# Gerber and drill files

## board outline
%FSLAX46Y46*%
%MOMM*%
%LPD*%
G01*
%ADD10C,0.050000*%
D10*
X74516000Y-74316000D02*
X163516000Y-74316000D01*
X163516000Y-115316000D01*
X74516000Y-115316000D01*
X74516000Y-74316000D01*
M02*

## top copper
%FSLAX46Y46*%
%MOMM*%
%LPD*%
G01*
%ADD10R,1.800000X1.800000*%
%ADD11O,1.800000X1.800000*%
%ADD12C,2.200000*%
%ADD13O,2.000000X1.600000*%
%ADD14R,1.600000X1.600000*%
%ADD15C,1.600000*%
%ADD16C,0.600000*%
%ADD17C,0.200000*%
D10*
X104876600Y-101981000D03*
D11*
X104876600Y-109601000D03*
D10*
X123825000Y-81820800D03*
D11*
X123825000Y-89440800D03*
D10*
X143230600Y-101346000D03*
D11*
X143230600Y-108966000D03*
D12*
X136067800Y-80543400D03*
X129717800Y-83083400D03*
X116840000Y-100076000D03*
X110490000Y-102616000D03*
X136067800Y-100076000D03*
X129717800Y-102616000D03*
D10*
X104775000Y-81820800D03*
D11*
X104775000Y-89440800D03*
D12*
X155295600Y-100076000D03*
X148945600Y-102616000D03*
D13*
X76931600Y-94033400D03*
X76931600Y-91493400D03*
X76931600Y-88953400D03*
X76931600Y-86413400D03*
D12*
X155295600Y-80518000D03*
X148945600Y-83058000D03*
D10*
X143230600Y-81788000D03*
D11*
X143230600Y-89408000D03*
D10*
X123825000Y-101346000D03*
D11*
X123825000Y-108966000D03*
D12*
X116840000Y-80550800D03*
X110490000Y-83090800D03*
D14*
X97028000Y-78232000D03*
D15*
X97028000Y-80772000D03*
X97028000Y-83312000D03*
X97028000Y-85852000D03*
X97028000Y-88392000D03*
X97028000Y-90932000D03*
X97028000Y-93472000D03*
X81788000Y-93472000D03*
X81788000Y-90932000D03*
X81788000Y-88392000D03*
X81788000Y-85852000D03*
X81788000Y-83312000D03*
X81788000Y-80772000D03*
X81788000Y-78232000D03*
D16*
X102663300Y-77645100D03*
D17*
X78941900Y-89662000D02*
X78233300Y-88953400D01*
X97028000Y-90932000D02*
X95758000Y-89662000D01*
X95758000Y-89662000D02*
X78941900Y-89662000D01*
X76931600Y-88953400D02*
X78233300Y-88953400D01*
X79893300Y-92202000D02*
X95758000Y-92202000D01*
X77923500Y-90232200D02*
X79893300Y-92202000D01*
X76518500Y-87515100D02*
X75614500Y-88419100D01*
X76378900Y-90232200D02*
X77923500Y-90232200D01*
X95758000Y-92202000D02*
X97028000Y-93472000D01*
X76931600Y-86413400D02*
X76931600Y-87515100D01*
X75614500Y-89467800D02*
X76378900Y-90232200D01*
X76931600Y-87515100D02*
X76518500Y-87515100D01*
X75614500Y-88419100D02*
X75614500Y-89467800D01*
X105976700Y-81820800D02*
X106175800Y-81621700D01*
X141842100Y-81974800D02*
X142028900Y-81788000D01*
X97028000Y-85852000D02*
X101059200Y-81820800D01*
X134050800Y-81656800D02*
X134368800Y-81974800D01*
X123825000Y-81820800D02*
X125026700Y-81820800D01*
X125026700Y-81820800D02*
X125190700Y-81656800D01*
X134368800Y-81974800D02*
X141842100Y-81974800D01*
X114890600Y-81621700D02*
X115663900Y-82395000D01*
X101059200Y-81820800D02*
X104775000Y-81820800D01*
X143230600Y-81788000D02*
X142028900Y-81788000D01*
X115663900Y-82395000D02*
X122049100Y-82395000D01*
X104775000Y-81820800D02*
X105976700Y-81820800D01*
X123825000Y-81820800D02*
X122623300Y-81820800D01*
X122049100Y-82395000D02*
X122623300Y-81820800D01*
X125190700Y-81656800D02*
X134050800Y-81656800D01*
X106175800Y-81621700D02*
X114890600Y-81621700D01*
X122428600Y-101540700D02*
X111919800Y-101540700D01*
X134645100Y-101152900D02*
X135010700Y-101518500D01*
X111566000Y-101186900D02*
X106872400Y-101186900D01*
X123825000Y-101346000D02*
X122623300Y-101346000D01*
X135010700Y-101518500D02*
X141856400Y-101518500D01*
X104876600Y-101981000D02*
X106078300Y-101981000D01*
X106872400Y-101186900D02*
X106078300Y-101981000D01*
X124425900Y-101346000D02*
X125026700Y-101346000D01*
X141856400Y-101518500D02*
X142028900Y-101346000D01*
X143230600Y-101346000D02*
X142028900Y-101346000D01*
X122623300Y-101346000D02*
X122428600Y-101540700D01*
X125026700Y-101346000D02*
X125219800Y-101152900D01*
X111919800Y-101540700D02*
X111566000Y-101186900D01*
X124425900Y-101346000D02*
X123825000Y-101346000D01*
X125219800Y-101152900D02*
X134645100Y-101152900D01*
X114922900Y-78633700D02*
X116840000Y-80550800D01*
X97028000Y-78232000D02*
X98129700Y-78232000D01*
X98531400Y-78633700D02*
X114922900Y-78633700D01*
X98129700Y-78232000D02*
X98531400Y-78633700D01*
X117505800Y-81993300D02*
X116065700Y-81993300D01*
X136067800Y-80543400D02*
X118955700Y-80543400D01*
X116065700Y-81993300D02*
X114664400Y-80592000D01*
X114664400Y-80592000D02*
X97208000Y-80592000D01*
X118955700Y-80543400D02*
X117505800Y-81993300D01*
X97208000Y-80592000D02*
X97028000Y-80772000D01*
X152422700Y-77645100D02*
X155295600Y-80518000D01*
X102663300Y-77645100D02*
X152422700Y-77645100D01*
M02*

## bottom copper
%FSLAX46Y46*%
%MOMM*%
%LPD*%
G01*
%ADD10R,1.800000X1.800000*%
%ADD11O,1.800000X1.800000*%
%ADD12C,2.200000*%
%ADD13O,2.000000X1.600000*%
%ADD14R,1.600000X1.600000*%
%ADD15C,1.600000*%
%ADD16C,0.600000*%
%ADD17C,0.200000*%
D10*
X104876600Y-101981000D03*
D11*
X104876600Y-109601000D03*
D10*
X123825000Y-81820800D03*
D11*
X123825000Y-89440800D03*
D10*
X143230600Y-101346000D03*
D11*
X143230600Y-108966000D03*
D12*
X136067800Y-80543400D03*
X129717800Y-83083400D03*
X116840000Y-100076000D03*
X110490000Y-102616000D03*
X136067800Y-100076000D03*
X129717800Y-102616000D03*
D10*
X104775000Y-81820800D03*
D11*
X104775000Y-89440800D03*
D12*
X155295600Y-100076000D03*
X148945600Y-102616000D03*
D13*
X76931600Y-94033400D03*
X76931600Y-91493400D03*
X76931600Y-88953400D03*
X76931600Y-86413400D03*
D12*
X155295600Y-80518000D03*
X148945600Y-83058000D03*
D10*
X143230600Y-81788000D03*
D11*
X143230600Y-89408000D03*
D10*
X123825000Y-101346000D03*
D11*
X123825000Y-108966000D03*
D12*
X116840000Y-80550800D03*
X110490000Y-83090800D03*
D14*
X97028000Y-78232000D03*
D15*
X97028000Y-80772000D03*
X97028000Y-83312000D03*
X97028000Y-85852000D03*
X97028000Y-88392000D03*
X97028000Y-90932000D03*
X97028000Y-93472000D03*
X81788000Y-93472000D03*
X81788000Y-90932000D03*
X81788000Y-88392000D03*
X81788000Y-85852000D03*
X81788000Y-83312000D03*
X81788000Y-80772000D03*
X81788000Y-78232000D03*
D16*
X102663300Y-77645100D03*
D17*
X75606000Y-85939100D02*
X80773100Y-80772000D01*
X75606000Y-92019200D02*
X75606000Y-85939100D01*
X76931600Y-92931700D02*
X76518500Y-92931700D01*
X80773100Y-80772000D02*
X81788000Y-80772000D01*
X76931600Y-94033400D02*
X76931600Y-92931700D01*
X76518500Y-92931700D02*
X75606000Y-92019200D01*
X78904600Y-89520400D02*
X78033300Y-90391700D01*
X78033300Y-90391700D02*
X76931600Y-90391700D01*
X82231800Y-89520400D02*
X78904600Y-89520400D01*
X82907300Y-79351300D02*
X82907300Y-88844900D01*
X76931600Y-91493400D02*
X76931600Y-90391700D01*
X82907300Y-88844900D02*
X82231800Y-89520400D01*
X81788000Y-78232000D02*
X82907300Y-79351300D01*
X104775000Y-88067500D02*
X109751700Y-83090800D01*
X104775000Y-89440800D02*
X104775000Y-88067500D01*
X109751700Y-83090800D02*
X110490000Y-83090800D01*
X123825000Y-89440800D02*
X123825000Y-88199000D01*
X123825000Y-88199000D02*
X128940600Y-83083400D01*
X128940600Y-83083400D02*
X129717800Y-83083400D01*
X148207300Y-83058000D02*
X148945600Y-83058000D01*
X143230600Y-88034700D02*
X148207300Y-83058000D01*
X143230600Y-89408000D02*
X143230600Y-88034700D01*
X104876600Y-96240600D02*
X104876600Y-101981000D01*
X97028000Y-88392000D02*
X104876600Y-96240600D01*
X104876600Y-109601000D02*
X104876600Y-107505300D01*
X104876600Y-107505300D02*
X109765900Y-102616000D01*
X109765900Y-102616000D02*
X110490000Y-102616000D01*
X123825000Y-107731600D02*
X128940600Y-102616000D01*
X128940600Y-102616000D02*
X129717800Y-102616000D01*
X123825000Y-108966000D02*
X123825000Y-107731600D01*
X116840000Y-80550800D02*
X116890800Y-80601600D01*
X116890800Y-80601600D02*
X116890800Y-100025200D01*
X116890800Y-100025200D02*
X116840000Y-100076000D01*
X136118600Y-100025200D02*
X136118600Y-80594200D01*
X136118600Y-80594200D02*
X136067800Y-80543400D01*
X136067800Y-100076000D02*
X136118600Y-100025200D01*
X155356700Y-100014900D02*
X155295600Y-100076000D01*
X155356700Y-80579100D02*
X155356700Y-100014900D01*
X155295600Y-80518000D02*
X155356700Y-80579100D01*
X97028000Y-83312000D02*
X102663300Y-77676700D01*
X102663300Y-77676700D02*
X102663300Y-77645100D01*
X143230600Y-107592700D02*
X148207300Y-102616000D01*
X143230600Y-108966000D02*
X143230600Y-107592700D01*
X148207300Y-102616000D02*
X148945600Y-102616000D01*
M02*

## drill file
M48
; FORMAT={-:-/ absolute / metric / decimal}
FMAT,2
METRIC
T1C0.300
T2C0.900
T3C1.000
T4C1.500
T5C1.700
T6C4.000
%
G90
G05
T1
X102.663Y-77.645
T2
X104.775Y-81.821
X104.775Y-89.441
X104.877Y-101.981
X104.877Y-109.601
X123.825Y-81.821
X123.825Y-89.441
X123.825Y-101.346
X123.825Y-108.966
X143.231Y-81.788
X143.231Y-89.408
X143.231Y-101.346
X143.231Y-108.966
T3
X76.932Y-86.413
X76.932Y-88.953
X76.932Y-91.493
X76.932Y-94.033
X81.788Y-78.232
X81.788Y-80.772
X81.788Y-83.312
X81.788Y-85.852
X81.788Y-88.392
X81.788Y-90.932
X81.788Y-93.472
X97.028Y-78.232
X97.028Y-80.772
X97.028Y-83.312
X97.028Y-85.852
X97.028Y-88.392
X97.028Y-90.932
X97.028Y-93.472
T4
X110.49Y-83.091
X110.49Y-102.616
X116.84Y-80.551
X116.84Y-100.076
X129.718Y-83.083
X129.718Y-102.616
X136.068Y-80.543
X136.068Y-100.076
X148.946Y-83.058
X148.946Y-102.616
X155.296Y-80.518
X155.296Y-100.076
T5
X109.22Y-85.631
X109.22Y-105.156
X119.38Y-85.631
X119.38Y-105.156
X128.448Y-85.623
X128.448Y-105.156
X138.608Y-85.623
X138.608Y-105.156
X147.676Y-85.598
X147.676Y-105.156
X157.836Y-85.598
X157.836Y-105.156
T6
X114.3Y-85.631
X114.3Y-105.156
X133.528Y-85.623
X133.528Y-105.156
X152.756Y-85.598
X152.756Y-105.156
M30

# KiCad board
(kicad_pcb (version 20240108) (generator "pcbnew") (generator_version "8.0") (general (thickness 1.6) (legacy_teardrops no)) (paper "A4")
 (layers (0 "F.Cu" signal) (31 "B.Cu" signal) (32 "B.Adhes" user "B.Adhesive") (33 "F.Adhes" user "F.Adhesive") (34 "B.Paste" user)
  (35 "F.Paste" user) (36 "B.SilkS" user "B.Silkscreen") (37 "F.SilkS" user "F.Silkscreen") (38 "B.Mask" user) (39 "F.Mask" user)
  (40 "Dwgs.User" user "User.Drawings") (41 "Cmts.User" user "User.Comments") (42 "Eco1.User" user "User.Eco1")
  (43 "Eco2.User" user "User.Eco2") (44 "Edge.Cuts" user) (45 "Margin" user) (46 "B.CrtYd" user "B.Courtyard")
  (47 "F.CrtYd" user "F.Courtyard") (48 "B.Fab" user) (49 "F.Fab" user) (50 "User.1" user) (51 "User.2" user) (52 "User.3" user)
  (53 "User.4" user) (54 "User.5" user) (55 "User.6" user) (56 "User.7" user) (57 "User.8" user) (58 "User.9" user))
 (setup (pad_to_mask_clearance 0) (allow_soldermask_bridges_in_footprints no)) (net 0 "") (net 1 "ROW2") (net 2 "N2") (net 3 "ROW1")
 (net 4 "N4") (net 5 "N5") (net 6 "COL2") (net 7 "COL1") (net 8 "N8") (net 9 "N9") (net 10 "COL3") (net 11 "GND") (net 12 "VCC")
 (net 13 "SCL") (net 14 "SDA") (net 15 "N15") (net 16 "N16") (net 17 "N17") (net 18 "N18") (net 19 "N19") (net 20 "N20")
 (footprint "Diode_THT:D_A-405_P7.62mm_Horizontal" (layer "F.Cu") (at 104.8766 101.981 -90)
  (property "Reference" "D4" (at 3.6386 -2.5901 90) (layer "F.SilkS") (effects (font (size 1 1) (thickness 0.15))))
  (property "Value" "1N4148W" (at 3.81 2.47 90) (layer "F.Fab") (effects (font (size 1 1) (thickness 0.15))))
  (pad "1" thru_hole rect (at 0 0 270) (size 1.8 1.8) (drill 0.9) (layers "*.Cu" "*.Mask") (remove_unused_layers no) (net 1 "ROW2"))
  (pad "2" thru_hole oval (at 7.62 0 270) (size 1.8 1.8) (drill 0.9) (layers "*.Cu" "*.Mask") (remove_unused_layers no) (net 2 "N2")))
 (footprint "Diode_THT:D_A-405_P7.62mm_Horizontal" (layer "F.Cu") (at 123.825 81.8208 -90)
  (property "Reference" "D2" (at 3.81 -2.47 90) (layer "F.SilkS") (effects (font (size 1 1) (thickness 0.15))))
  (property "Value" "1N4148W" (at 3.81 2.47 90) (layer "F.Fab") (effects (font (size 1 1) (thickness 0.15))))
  (pad "1" thru_hole rect (at 0 0 270) (size 1.8 1.8) (drill 0.9) (layers "*.Cu" "*.Mask") (remove_unused_layers no) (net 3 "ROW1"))
  (pad "2" thru_hole oval (at 7.62 0 270) (size 1.8 1.8) (drill 0.9) (layers "*.Cu" "*.Mask") (remove_unused_layers no) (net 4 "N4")))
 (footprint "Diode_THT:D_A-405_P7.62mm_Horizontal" (layer "F.Cu") (at 143.2306 101.346 -90)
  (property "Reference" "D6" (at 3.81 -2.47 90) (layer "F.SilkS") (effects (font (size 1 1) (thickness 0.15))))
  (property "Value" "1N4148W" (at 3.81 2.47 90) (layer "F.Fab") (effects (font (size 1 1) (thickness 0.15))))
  (pad "1" thru_hole rect (at 0 0 270) (size 1.8 1.8) (drill 0.9) (layers "*.Cu" "*.Mask") (remove_unused_layers no) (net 1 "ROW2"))
  (pad "2" thru_hole oval (at 7.62 0 270) (size 1.8 1.8) (drill 0.9) (layers "*.Cu" "*.Mask") (remove_unused_layers no) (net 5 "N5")))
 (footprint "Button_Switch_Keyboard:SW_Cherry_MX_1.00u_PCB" (layer "F.Cu") (at 136.0678 80.5434)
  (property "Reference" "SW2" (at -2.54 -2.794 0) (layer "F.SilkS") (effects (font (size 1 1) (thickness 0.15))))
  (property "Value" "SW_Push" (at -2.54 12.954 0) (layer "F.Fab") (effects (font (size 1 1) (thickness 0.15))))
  (pad "" np_thru_hole circle (at -7.62 5.08) (size 1.7 1.7) (drill 1.7) (layers "*.Cu" "*.Mask"))
  (pad "" np_thru_hole circle (at -2.54 5.08) (size 4 4) (drill 4) (layers "*.Cu" "*.Mask"))
  (pad "" np_thru_hole circle (at 2.54 5.08) (size 1.7 1.7) (drill 1.7) (layers "*.Cu" "*.Mask"))
  (pad "1" thru_hole circle (at 0 0) (size 2.2 2.2) (drill 1.5) (layers "*.Cu" "*.Mask") (remove_unused_layers no) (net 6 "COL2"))
  (pad "2" thru_hole circle (at -6.35 2.54) (size 2.2 2.2) (drill 1.5) (layers "*.Cu" "*.Mask") (remove_unused_layers no) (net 4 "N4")))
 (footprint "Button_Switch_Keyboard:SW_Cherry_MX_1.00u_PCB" (layer "F.Cu") (at 116.84 100.076)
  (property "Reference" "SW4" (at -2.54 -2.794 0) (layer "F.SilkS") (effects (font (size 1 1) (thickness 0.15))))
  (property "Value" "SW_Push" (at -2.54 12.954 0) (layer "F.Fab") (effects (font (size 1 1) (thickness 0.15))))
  (pad "" np_thru_hole circle (at -7.62 5.08) (size 1.7 1.7) (drill 1.7) (layers "*.Cu" "*.Mask"))
  (pad "" np_thru_hole circle (at -2.54 5.08) (size 4 4) (drill 4) (layers "*.Cu" "*.Mask"))
  (pad "" np_thru_hole circle (at 2.54 5.08) (size 1.7 1.7) (drill 1.7) (layers "*.Cu" "*.Mask"))
  (pad "1" thru_hole circle (at 0 0) (size 2.2 2.2) (drill 1.5) (layers "*.Cu" "*.Mask") (remove_unused_layers no) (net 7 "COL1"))
  (pad "2" thru_hole circle (at -6.35 2.54) (size 2.2 2.2) (drill 1.5) (layers "*.Cu" "*.Mask") (remove_unused_layers no) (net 2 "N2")))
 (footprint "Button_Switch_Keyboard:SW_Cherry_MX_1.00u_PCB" (layer "F.Cu") (at 136.0678 100.076)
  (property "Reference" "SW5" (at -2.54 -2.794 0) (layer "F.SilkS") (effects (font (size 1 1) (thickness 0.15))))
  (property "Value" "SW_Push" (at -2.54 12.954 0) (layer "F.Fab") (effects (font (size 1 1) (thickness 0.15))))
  (pad "" np_thru_hole circle (at -7.62 5.08) (size 1.7 1.7) (drill 1.7) (layers "*.Cu" "*.Mask"))
  (pad "" np_thru_hole circle (at -2.54 5.08) (size 4 4) (drill 4) (layers "*.Cu" "*.Mask"))
  (pad "" np_thru_hole circle (at 2.54 5.08) (size 1.7 1.7) (drill 1.7) (layers "*.Cu" "*.Mask"))
  (pad "1" thru_hole circle (at 0 0) (size 2.2 2.2) (drill 1.5) (layers "*.Cu" "*.Mask") (remove_unused_layers no) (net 6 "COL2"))
  (pad "2" thru_hole circle (at -6.35 2.54) (size 2.2 2.2) (drill 1.5) (layers "*.Cu" "*.Mask") (remove_unused_layers no) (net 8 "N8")))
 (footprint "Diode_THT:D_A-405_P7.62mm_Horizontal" (layer "F.Cu") (at 104.775 81.8208 -90)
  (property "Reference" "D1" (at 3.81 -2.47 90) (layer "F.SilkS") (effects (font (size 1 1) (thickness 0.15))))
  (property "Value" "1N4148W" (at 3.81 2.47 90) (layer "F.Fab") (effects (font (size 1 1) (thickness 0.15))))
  (pad "1" thru_hole rect (at 0 0 270) (size 1.8 1.8) (drill 0.9) (layers "*.Cu" "*.Mask") (remove_unused_layers no) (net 3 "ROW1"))
  (pad "2" thru_hole oval (at 7.62 0 270) (size 1.8 1.8) (drill 0.9) (layers "*.Cu" "*.Mask") (remove_unused_layers no) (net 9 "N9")))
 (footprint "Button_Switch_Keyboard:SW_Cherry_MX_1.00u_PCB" (layer "F.Cu") (at 155.2956 100.076)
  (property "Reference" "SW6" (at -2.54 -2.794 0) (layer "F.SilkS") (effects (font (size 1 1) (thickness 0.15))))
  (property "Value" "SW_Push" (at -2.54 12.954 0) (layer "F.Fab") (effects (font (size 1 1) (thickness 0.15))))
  (pad "" np_thru_hole circle (at -7.62 5.08) (size 1.7 1.7) (drill 1.7) (layers "*.Cu" "*.Mask"))
  (pad "" np_thru_hole circle (at -2.54 5.08) (size 4 4) (drill 4) (layers "*.Cu" "*.Mask"))
  (pad "" np_thru_hole circle (at 2.54 5.08) (size 1.7 1.7) (drill 1.7) (layers "*.Cu" "*.Mask"))
  (pad "1" thru_hole circle (at 0 0) (size 2.2 2.2) (drill 1.5) (layers "*.Cu" "*.Mask") (remove_unused_layers no) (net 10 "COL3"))
  (pad "2" thru_hole circle (at -6.35 2.54) (size 2.2 2.2) (drill 1.5) (layers "*.Cu" "*.Mask") (remove_unused_layers no) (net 5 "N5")))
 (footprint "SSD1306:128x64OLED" (layer "F.Cu") (at 87.5316 90.4134 90)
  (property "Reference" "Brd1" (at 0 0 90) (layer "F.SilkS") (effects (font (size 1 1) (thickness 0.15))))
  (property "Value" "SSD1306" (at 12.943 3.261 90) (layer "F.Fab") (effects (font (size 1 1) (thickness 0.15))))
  (pad "1" thru_hole oval (at -3.62 -10.6 180) (size 2 1.6) (drill 1) (layers "*.Cu" "*.Mask") (remove_unused_layers no) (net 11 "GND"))
  (pad "2" thru_hole oval (at -1.08 -10.6 180) (size 2 1.6) (drill 1) (layers "*.Cu" "*.Mask") (remove_unused_layers no) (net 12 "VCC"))
  (pad "3" thru_hole oval (at 1.46 -10.6 180) (size 2 1.6) (drill 1) (layers "*.Cu" "*.Mask") (remove_unused_layers no) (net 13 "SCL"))
  (pad "4" thru_hole oval (at 4 -10.6 180) (size 2 1.6) (drill 1) (layers "*.Cu" "*.Mask") (remove_unused_layers no) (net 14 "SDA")))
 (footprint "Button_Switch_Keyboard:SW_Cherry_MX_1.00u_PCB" (layer "F.Cu") (at 155.2956 80.518)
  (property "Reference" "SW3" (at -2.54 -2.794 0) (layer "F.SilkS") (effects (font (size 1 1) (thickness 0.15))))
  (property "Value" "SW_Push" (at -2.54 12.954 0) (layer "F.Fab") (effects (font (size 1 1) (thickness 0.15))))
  (pad "" np_thru_hole circle (at -7.62 5.08) (size 1.7 1.7) (drill 1.7) (layers "*.Cu" "*.Mask"))
  (pad "" np_thru_hole circle (at -2.54 5.08) (size 4 4) (drill 4) (layers "*.Cu" "*.Mask"))
  (pad "" np_thru_hole circle (at 2.54 5.08) (size 1.7 1.7) (drill 1.7) (layers "*.Cu" "*.Mask"))
  (pad "1" thru_hole circle (at 0 0) (size 2.2 2.2) (drill 1.5) (layers "*.Cu" "*.Mask") (remove_unused_layers no) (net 10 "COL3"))
  (pad "2" thru_hole circle (at -6.35 2.54) (size 2.2 2.2) (drill 1.5) (layers "*.Cu" "*.Mask") (remove_unused_layers no) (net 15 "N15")))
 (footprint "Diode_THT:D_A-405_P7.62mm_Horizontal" (layer "F.Cu") (at 143.2306 81.788 -90)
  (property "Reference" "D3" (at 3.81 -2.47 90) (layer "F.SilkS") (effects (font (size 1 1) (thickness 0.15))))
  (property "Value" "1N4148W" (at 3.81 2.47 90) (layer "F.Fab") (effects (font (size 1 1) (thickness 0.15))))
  (pad "1" thru_hole rect (at 0 0 270) (size 1.8 1.8) (drill 0.9) (layers "*.Cu" "*.Mask") (remove_unused_layers no) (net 3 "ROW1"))
  (pad "2" thru_hole oval (at 7.62 0 270) (size 1.8 1.8) (drill 0.9) (layers "*.Cu" "*.Mask") (remove_unused_layers no) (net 15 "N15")))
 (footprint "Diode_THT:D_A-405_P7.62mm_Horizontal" (layer "F.Cu") (at 123.825 101.346 -90)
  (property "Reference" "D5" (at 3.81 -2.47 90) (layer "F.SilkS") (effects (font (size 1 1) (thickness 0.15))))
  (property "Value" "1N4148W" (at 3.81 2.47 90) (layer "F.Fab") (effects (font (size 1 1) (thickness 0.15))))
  (pad "1" thru_hole rect (at 0 0 270) (size 1.8 1.8) (drill 0.9) (layers "*.Cu" "*.Mask") (remove_unused_layers no) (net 1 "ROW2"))
  (pad "2" thru_hole oval (at 7.62 0 270) (size 1.8 1.8) (drill 0.9) (layers "*.Cu" "*.Mask") (remove_unused_layers no) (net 8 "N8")))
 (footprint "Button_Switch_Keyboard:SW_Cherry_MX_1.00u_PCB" (layer "F.Cu") (at 116.84 80.5508)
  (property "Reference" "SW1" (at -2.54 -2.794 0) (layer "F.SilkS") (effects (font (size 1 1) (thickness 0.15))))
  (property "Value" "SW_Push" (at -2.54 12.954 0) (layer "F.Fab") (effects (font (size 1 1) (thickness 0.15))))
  (pad "" np_thru_hole circle (at -7.62 5.08) (size 1.7 1.7) (drill 1.7) (layers "*.Cu" "*.Mask"))
  (pad "" np_thru_hole circle (at -2.54 5.08) (size 4 4) (drill 4) (layers "*.Cu" "*.Mask"))
  (pad "" np_thru_hole circle (at 2.54 5.08) (size 1.7 1.7) (drill 1.7) (layers "*.Cu" "*.Mask"))
  (pad "1" thru_hole circle (at 0 0) (size 2.2 2.2) (drill 1.5) (layers "*.Cu" "*.Mask") (remove_unused_layers no) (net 7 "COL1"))
  (pad "2" thru_hole circle (at -6.35 2.54) (size 2.2 2.2) (drill 1.5) (layers "*.Cu" "*.Mask") (remove_unused_layers no) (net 9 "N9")))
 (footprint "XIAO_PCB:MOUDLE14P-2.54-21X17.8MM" (layer "B.Cu") (at 89.408 85.852 90)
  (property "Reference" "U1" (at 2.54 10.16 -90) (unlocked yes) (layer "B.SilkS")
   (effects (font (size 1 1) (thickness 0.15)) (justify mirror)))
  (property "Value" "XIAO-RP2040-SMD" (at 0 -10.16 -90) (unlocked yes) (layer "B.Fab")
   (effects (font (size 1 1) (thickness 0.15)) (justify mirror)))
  (pad "1" thru_hole rect (at 7.62 7.62 90) (size 1.6 1.6) (drill 1) (layers "*.Cu" "*.Mask") (remove_unused_layers no) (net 7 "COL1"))
  (pad "2" thru_hole circle (at 5.08 7.62 90) (size 1.6 1.6) (drill 1) (layers "*.Cu" "*.Mask") (remove_unused_layers no) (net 6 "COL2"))
  (pad "3" thru_hole circle (at 2.54 7.62 90) (size 1.6 1.6) (drill 1) (layers "*.Cu" "*.Mask") (remove_unused_layers no) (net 10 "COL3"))
  (pad "4" thru_hole circle (at 0 7.62 90) (size 1.6 1.6) (drill 1) (layers "*.Cu" "*.Mask") (remove_unused_layers no) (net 3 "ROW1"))
  (pad "5" thru_hole circle (at -2.54 7.62 90) (size 1.6 1.6) (drill 1) (layers "*.Cu" "*.Mask") (remove_unused_layers no) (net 1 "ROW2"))
  (pad "6" thru_hole circle (at -5.08 7.62 90) (size 1.6 1.6) (drill 1) (layers "*.Cu" "*.Mask") (remove_unused_layers no) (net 13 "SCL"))
  (pad "7" thru_hole circle (at -7.62 7.62 90) (size 1.6 1.6) (drill 1) (layers "*.Cu" "*.Mask") (remove_unused_layers no) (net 14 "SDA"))
  (pad "8" thru_hole circle (at -7.62 -7.62 90) (size 1.6 1.6) (drill 1) (layers "*.Cu" "*.Mask") (remove_unused_layers no) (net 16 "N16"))
  (pad "9" thru_hole circle (at -5.08 -7.62 90) (size 1.6 1.6) (drill 1) (layers "*.Cu" "*.Mask") (remove_unused_layers no) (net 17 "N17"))
  (pad "10" thru_hole circle (at -2.54 -7.62 90) (size 1.6 1.6) (drill 1) (layers "*.Cu" "*.Mask") (remove_unused_layers no) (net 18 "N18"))
  (pad "11" thru_hole circle (at 0 -7.62 90) (size 1.6 1.6) (drill 1) (layers "*.Cu" "*.Mask") (remove_unused_layers no) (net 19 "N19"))
  (pad "12" thru_hole circle (at 2.54 -7.62 90) (size 1.6 1.6) (drill 1) (layers "*.Cu" "*.Mask") (remove_unused_layers no) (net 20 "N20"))
  (pad "13" thru_hole circle (at 5.08 -7.62 90) (size 1.6 1.6) (drill 1) (layers "*.Cu" "*.Mask") (remove_unused_layers no) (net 11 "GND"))
  (pad "14" thru_hole circle (at 7.62 -7.62 90) (size 1.6 1.6) (drill 1) (layers "*.Cu" "*.Mask") (remove_unused_layers no) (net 12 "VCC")))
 (gr_rect (start 74.516 74.316) (end 163.516 115.316) (stroke (width 0.05) (type default)) (fill none) (layer "Edge.Cuts"))
 (segment (start 78.9419 89.662) (end 78.2333 88.9534) (width 0.2) (layer "F.Cu") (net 13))
 (segment (start 97.028 90.932) (end 95.758 89.662) (width 0.2) (layer "F.Cu") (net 13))
 (segment (start 95.758 89.662) (end 78.9419 89.662) (width 0.2) (layer "F.Cu") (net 13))
 (segment (start 76.9316 88.9534) (end 78.2333 88.9534) (width 0.2) (layer "F.Cu") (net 13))
 (segment (start 75.606 85.9391) (end 80.7731 80.772) (width 0.2) (layer "B.Cu") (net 11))
 (segment (start 75.606 92.0192) (end 75.606 85.9391) (width 0.2) (layer "B.Cu") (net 11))
 (segment (start 76.9316 92.9317) (end 76.5185 92.9317) (width 0.2) (layer "B.Cu") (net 11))
 (segment (start 80.7731 80.772) (end 81.788 80.772) (width 0.2) (layer "B.Cu") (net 11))
 (segment (start 76.9316 94.0334) (end 76.9316 92.9317) (width 0.2) (layer "B.Cu") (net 11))
 (segment (start 76.5185 92.9317) (end 75.606 92.0192) (width 0.2) (layer "B.Cu") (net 11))
 (segment (start 78.9046 89.5204) (end 78.0333 90.3917) (width 0.2) (layer "B.Cu") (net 12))
 (segment (start 78.0333 90.3917) (end 76.9316 90.3917) (width 0.2) (layer "B.Cu") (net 12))
 (segment (start 82.2318 89.5204) (end 78.9046 89.5204) (width 0.2) (layer "B.Cu") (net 12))
 (segment (start 82.9073 79.3513) (end 82.9073 88.8449) (width 0.2) (layer "B.Cu") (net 12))
 (segment (start 76.9316 91.4934) (end 76.9316 90.3917) (width 0.2) (layer "B.Cu") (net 12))
 (segment (start 82.9073 88.8449) (end 82.2318 89.5204) (width 0.2) (layer "B.Cu") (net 12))
 (segment (start 81.788 78.232) (end 82.9073 79.3513) (width 0.2) (layer "B.Cu") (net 12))
 (segment (start 79.8933 92.202) (end 95.758 92.202) (width 0.2) (layer "F.Cu") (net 14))
 (segment (start 77.9235 90.2322) (end 79.8933 92.202) (width 0.2) (layer "F.Cu") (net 14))
 (segment (start 76.5185 87.5151) (end 75.6145 88.4191) (width 0.2) (layer "F.Cu") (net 14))
 (segment (start 76.3789 90.2322) (end 77.9235 90.2322) (width 0.2) (layer "F.Cu") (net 14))
 (segment (start 95.758 92.202) (end 97.028 93.472) (width 0.2) (layer "F.Cu") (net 14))
 (segment (start 76.9316 86.4134) (end 76.9316 87.5151) (width 0.2) (layer "F.Cu") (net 14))
 (segment (start 75.6145 89.4678) (end 76.3789 90.2322) (width 0.2) (layer "F.Cu") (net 14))
 (segment (start 76.9316 87.5151) (end 76.5185 87.5151) (width 0.2) (layer "F.Cu") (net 14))
 (segment (start 75.6145 88.4191) (end 75.6145 89.4678) (width 0.2) (layer "F.Cu") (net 14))
 (segment (start 104.775 88.0675) (end 109.7517 83.0908) (width 0.2) (layer "B.Cu") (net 9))
 (segment (start 104.775 89.4408) (end 104.775 88.0675) (width 0.2) (layer "B.Cu") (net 9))
 (segment (start 109.7517 83.0908) (end 110.49 83.0908) (width 0.2) (layer "B.Cu") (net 9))
 (segment (start 105.9767 81.8208) (end 106.1758 81.6217) (width 0.2) (layer "F.Cu") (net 3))
 (segment (start 141.8421 81.9748) (end 142.0289 81.788) (width 0.2) (layer "F.Cu") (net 3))
 (segment (start 97.028 85.852) (end 101.0592 81.8208) (width 0.2) (layer "F.Cu") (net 3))
 (segment (start 134.0508 81.6568) (end 134.3688 81.9748) (width 0.2) (layer "F.Cu") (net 3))
 (segment (start 123.825 81.8208) (end 125.0267 81.8208) (width 0.2) (layer "F.Cu") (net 3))
 (segment (start 125.0267 81.8208) (end 125.1907 81.6568) (width 0.2) (layer "F.Cu") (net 3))
 (segment (start 134.3688 81.9748) (end 141.8421 81.9748) (width 0.2) (layer "F.Cu") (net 3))
 (segment (start 114.8906 81.6217) (end 115.6639 82.395) (width 0.2) (layer "F.Cu") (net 3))
 (segment (start 101.0592 81.8208) (end 104.775 81.8208) (width 0.2) (layer "F.Cu") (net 3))
 (segment (start 143.2306 81.788) (end 142.0289 81.788) (width 0.2) (layer "F.Cu") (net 3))
 (segment (start 115.6639 82.395) (end 122.0491 82.395) (width 0.2) (layer "F.Cu") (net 3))
 (segment (start 104.775 81.8208) (end 105.9767 81.8208) (width 0.2) (layer "F.Cu") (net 3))
 (segment (start 123.825 81.8208) (end 122.6233 81.8208) (width 0.2) (layer "F.Cu") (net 3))
 (segment (start 122.0491 82.395) (end 122.6233 81.8208) (width 0.2) (layer "F.Cu") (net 3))
 (segment (start 125.1907 81.6568) (end 134.0508 81.6568) (width 0.2) (layer "F.Cu") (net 3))
 (segment (start 106.1758 81.6217) (end 114.8906 81.6217) (width 0.2) (layer "F.Cu") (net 3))
 (segment (start 123.825 89.4408) (end 123.825 88.199) (width 0.2) (layer "B.Cu") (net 4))
 (segment (start 123.825 88.199) (end 128.9406 83.0834) (width 0.2) (layer "B.Cu") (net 4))
 (segment (start 128.9406 83.0834) (end 129.7178 83.0834) (width 0.2) (layer "B.Cu") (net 4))
 (segment (start 148.2073 83.058) (end 148.9456 83.058) (width 0.2) (layer "B.Cu") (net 15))
 (segment (start 143.2306 88.0347) (end 148.2073 83.058) (width 0.2) (layer "B.Cu") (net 15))
 (segment (start 143.2306 89.408) (end 143.2306 88.0347) (width 0.2) (layer "B.Cu") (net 15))
 (segment (start 122.4286 101.5407) (end 111.9198 101.5407) (width 0.2) (layer "F.Cu") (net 1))
 (segment (start 134.6451 101.1529) (end 135.0107 101.5185) (width 0.2) (layer "F.Cu") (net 1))
 (segment (start 111.566 101.1869) (end 106.8724 101.1869) (width 0.2) (layer "F.Cu") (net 1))
 (segment (start 123.825 101.346) (end 122.6233 101.346) (width 0.2) (layer "F.Cu") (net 1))
 (segment (start 135.0107 101.5185) (end 141.8564 101.5185) (width 0.2) (layer "F.Cu") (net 1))
 (segment (start 104.8766 101.981) (end 106.0783 101.981) (width 0.2) (layer "F.Cu") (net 1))
 (segment (start 106.8724 101.1869) (end 106.0783 101.981) (width 0.2) (layer "F.Cu") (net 1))
 (segment (start 124.4259 101.346) (end 125.0267 101.346) (width 0.2) (layer "F.Cu") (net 1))
 (segment (start 141.8564 101.5185) (end 142.0289 101.346) (width 0.2) (layer "F.Cu") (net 1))
 (segment (start 143.2306 101.346) (end 142.0289 101.346) (width 0.2) (layer "F.Cu") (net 1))
 (segment (start 122.6233 101.346) (end 122.4286 101.5407) (width 0.2) (layer "F.Cu") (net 1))
 (segment (start 125.0267 101.346) (end 125.2198 101.1529) (width 0.2) (layer "F.Cu") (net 1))
 (segment (start 111.9198 101.5407) (end 111.566 101.1869) (width 0.2) (layer "F.Cu") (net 1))
 (segment (start 124.4259 101.346) (end 123.825 101.346) (width 0.2) (layer "F.Cu") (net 1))
 (segment (start 125.2198 101.1529) (end 134.6451 101.1529) (width 0.2) (layer "F.Cu") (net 1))
 (segment (start 104.8766 96.2406) (end 104.8766 101.981) (width 0.2) (layer "B.Cu") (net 1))
 (segment (start 97.028 88.392) (end 104.8766 96.2406) (width 0.2) (layer "B.Cu") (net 1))
 (segment (start 104.8766 109.601) (end 104.8766 107.5053) (width 0.2) (layer "B.Cu") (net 2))
 (segment (start 104.8766 107.5053) (end 109.7659 102.616) (width 0.2) (layer "B.Cu") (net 2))
 (segment (start 109.7659 102.616) (end 110.49 102.616) (width 0.2) (layer "B.Cu") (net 2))
 (segment (start 123.825 107.7316) (end 128.9406 102.616) (width 0.2) (layer "B.Cu") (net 8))
 (segment (start 128.9406 102.616) (end 129.7178 102.616) (width 0.2) (layer "B.Cu") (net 8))
 (segment (start 123.825 108.966) (end 123.825 107.7316) (width 0.2) (layer "B.Cu") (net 8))
 (segment (start 114.9229 78.6337) (end 116.84 80.5508) (width 0.2) (layer "F.Cu") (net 7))
 (segment (start 97.028 78.232) (end 98.1297 78.232) (width 0.2) (layer "F.Cu") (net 7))
 (segment (start 98.5314 78.6337) (end 114.9229 78.6337) (width 0.2) (layer "F.Cu") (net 7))
 (segment (start 98.1297 78.232) (end 98.5314 78.6337) (width 0.2) (layer "F.Cu") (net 7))
 (segment (start 116.84 80.5508) (end 116.8908 80.6016) (width 0.2) (layer "B.Cu") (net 7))
 (segment (start 116.8908 80.6016) (end 116.8908 100.0252) (width 0.2) (layer "B.Cu") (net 7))
 (segment (start 116.8908 100.0252) (end 116.84 100.076) (width 0.2) (layer "B.Cu") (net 7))
 (segment (start 117.5058 81.9933) (end 116.0657 81.9933) (width 0.2) (layer "F.Cu") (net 6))
 (segment (start 136.0678 80.5434) (end 118.9557 80.5434) (width 0.2) (layer "F.Cu") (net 6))
 (segment (start 116.0657 81.9933) (end 114.6644 80.592) (width 0.2) (layer "F.Cu") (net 6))
 (segment (start 114.6644 80.592) (end 97.208 80.592) (width 0.2) (layer "F.Cu") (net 6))
 (segment (start 118.9557 80.5434) (end 117.5058 81.9933) (width 0.2) (layer "F.Cu") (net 6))
 (segment (start 97.208 80.592) (end 97.028 80.772) (width 0.2) (layer "F.Cu") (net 6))
 (segment (start 136.1186 100.0252) (end 136.1186 80.5942) (width 0.2) (layer "B.Cu") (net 6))
 (segment (start 136.1186 80.5942) (end 136.0678 80.5434) (width 0.2) (layer "B.Cu") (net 6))
 (segment (start 136.0678 100.076) (end 136.1186 100.0252) (width 0.2) (layer "B.Cu") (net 6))
 (segment (start 152.4227 77.6451) (end 155.2956 80.518) (width 0.2) (layer "F.Cu") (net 10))
 (segment (start 102.6633 77.6451) (end 152.4227 77.6451) (width 0.2) (layer "F.Cu") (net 10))
 (via (at 102.6633 77.6451) (size 0.6) (drill 0.3) (layers "F.Cu" "B.Cu") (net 10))
 (segment (start 155.3567 100.0149) (end 155.2956 100.076) (width 0.2) (layer "B.Cu") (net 10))
 (segment (start 155.3567 80.5791) (end 155.3567 100.0149) (width 0.2) (layer "B.Cu") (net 10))
 (segment (start 155.2956 80.518) (end 155.3567 80.5791) (width 0.2) (layer "B.Cu") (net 10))
 (segment (start 97.028 83.312) (end 102.6633 77.6767) (width 0.2) (layer "B.Cu") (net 10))
 (segment (start 102.6633 77.6767) (end 102.6633 77.6451) (width 0.2) (layer "B.Cu") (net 10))
 (segment (start 143.2306 107.5927) (end 148.2073 102.616) (width 0.2) (layer "B.Cu") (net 5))
 (segment (start 143.2306 108.966) (end 143.2306 107.5927) (width 0.2) (layer "B.Cu") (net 5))
 (segment (start 148.2073 102.616) (end 148.9456 102.616) (width 0.2) (layer "B.Cu") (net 5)))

